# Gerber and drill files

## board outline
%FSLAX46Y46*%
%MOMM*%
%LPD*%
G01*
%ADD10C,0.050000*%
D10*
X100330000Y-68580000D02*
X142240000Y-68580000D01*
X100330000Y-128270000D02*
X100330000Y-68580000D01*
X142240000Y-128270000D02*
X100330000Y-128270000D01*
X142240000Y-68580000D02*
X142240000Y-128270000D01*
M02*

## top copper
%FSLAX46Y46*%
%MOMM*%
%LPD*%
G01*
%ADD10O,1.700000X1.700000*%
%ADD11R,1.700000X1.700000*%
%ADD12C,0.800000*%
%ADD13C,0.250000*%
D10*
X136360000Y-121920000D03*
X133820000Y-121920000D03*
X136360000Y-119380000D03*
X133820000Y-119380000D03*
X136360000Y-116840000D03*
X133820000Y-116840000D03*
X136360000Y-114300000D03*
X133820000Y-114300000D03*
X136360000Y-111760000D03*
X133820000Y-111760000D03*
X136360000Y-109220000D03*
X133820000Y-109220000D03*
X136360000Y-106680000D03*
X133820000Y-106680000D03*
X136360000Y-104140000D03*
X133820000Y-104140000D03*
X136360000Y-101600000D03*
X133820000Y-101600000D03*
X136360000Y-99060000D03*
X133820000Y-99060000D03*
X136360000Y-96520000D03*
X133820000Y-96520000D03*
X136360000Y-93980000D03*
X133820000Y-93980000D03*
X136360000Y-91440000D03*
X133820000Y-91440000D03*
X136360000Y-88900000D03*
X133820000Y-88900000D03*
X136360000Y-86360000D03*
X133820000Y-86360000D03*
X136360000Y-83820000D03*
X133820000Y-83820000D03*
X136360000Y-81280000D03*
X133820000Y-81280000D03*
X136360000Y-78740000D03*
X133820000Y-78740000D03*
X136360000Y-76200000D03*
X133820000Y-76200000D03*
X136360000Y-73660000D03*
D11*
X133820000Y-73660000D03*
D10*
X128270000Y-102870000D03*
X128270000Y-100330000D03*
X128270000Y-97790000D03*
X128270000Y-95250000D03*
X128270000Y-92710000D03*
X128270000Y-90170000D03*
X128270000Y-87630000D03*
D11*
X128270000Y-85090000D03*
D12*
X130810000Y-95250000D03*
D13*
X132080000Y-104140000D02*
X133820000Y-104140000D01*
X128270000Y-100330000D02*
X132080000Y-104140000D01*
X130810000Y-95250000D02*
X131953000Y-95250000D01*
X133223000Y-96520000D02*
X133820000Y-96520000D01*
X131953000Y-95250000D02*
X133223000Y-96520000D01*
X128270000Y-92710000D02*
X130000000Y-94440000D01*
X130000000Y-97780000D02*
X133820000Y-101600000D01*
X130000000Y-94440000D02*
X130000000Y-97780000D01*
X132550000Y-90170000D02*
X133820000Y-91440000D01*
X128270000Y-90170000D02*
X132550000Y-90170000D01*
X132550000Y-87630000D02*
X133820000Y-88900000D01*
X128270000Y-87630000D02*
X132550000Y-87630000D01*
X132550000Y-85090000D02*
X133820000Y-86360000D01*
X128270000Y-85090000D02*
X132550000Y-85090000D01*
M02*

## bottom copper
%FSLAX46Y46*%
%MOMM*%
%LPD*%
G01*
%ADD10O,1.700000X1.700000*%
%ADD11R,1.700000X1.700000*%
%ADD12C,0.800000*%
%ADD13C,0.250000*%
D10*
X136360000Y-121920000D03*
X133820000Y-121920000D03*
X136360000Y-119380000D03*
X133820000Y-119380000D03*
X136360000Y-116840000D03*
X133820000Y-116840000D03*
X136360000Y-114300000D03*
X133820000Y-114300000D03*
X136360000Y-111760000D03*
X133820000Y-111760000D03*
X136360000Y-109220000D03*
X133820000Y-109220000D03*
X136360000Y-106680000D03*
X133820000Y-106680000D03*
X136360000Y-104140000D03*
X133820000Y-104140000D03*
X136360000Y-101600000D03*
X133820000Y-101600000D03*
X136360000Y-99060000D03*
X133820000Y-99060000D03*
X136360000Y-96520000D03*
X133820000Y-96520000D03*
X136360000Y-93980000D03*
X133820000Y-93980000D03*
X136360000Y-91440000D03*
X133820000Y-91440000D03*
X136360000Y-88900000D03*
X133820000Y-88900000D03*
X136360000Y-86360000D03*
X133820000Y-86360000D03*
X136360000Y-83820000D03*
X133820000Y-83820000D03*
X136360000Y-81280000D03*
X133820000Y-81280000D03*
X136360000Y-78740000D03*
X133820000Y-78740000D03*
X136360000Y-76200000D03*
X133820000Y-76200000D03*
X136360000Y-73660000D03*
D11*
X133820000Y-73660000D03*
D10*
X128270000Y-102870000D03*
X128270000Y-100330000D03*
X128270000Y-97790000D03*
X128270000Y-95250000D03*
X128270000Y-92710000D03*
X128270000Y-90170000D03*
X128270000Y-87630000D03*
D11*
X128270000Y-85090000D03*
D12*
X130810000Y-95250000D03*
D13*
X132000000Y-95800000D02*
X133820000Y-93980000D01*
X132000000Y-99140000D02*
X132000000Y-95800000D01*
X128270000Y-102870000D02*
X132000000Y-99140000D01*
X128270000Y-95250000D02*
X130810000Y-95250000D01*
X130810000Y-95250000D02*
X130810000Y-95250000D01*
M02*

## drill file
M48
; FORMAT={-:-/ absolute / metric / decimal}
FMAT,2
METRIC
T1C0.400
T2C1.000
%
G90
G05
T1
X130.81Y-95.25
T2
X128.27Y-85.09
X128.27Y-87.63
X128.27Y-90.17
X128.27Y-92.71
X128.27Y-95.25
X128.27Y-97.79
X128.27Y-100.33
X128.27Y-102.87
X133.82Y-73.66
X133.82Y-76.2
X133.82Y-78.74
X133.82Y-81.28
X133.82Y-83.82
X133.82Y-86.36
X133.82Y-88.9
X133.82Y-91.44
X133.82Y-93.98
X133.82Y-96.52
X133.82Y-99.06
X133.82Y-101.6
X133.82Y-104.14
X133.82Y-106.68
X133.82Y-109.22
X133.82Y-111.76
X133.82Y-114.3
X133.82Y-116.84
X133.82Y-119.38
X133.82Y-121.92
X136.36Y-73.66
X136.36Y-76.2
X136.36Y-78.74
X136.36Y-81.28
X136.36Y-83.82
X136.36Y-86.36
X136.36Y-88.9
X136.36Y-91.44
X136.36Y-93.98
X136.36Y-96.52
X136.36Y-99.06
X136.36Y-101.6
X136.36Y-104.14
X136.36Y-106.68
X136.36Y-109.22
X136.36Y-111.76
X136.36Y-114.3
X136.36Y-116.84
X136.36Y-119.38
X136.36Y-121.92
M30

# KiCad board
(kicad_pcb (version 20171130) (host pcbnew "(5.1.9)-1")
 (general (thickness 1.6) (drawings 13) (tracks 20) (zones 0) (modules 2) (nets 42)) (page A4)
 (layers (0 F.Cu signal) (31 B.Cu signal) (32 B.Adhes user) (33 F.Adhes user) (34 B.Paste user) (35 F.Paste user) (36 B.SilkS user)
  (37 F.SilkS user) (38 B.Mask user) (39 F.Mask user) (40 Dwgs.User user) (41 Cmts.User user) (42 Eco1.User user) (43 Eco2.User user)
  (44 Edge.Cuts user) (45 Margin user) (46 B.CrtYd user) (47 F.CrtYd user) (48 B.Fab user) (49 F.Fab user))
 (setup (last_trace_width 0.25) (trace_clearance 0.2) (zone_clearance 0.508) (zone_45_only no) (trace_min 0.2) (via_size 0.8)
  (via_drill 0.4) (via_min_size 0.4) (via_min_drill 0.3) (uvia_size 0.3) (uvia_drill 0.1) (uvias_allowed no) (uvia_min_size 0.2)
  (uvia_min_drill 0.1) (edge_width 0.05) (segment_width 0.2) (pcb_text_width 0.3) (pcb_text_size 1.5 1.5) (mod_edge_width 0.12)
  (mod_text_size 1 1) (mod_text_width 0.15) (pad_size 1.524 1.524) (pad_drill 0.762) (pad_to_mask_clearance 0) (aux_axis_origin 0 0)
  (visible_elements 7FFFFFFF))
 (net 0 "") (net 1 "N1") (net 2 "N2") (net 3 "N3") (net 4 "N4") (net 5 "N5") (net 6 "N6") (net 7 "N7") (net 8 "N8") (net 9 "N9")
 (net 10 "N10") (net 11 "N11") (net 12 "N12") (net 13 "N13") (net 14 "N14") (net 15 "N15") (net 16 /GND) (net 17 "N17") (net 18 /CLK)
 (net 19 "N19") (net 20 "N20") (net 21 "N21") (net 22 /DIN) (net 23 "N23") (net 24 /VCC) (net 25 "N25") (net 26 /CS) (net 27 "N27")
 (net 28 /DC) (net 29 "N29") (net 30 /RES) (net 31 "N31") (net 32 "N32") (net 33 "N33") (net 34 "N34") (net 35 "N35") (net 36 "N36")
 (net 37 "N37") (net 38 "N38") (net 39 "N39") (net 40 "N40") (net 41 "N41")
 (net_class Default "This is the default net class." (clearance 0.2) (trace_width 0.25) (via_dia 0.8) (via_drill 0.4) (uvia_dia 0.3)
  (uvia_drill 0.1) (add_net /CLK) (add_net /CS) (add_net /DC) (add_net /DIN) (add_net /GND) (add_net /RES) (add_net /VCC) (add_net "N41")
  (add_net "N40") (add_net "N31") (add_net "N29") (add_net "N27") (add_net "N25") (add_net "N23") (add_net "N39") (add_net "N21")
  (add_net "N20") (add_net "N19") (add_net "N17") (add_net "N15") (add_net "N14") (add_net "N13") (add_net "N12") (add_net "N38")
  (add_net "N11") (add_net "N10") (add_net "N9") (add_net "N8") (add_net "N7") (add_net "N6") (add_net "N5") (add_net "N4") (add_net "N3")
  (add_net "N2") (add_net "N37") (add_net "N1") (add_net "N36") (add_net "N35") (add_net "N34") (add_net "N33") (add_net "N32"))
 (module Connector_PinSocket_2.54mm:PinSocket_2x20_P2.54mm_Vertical (layer B.Cu) (at 133.82 73.66 180)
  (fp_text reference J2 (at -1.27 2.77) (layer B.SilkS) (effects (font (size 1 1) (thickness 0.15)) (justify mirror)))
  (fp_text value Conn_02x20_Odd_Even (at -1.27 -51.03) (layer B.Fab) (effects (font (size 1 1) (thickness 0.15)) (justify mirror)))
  (pad 40 thru_hole oval (at -2.54 -48.26 180) (size 1.7 1.7) (drill 1) (layers *.Cu *.Mask) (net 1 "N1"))
  (pad 39 thru_hole oval (at 0 -48.26 180) (size 1.7 1.7) (drill 1) (layers *.Cu *.Mask) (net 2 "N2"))
  (pad 38 thru_hole oval (at -2.54 -45.72 180) (size 1.7 1.7) (drill 1) (layers *.Cu *.Mask) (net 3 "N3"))
  (pad 37 thru_hole oval (at 0 -45.72 180) (size 1.7 1.7) (drill 1) (layers *.Cu *.Mask) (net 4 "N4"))
  (pad 36 thru_hole oval (at -2.54 -43.18 180) (size 1.7 1.7) (drill 1) (layers *.Cu *.Mask) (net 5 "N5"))
  (pad 35 thru_hole oval (at 0 -43.18 180) (size 1.7 1.7) (drill 1) (layers *.Cu *.Mask) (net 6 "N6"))
  (pad 34 thru_hole oval (at -2.54 -40.64 180) (size 1.7 1.7) (drill 1) (layers *.Cu *.Mask) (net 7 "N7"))
  (pad 33 thru_hole oval (at 0 -40.64 180) (size 1.7 1.7) (drill 1) (layers *.Cu *.Mask) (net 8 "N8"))
  (pad 32 thru_hole oval (at -2.54 -38.1 180) (size 1.7 1.7) (drill 1) (layers *.Cu *.Mask) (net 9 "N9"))
  (pad 31 thru_hole oval (at 0 -38.1 180) (size 1.7 1.7) (drill 1) (layers *.Cu *.Mask) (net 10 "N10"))
  (pad 30 thru_hole oval (at -2.54 -35.56 180) (size 1.7 1.7) (drill 1) (layers *.Cu *.Mask) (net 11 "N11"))
  (pad 29 thru_hole oval (at 0 -35.56 180) (size 1.7 1.7) (drill 1) (layers *.Cu *.Mask) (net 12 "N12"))
  (pad 28 thru_hole oval (at -2.54 -33.02 180) (size 1.7 1.7) (drill 1) (layers *.Cu *.Mask) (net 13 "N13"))
  (pad 27 thru_hole oval (at 0 -33.02 180) (size 1.7 1.7) (drill 1) (layers *.Cu *.Mask) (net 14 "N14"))
  (pad 26 thru_hole oval (at -2.54 -30.48 180) (size 1.7 1.7) (drill 1) (layers *.Cu *.Mask) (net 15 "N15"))
  (pad 25 thru_hole oval (at 0 -30.48 180) (size 1.7 1.7) (drill 1) (layers *.Cu *.Mask) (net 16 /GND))
  (pad 24 thru_hole oval (at -2.54 -27.94 180) (size 1.7 1.7) (drill 1) (layers *.Cu *.Mask) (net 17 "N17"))
  (pad 23 thru_hole oval (at 0 -27.94 180) (size 1.7 1.7) (drill 1) (layers *.Cu *.Mask) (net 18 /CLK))
  (pad 22 thru_hole oval (at -2.54 -25.4 180) (size 1.7 1.7) (drill 1) (layers *.Cu *.Mask) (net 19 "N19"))
  (pad 21 thru_hole oval (at 0 -25.4 180) (size 1.7 1.7) (drill 1) (layers *.Cu *.Mask) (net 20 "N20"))
  (pad 20 thru_hole oval (at -2.54 -22.86 180) (size 1.7 1.7) (drill 1) (layers *.Cu *.Mask) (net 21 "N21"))
  (pad 19 thru_hole oval (at 0 -22.86 180) (size 1.7 1.7) (drill 1) (layers *.Cu *.Mask) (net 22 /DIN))
  (pad 18 thru_hole oval (at -2.54 -20.32 180) (size 1.7 1.7) (drill 1) (layers *.Cu *.Mask) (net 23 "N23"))
  (pad 17 thru_hole oval (at 0 -20.32 180) (size 1.7 1.7) (drill 1) (layers *.Cu *.Mask) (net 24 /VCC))
  (pad 16 thru_hole oval (at -2.54 -17.78 180) (size 1.7 1.7) (drill 1) (layers *.Cu *.Mask) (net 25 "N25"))
  (pad 15 thru_hole oval (at 0 -17.78 180) (size 1.7 1.7) (drill 1) (layers *.Cu *.Mask) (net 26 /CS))
  (pad 14 thru_hole oval (at -2.54 -15.24 180) (size 1.7 1.7) (drill 1) (layers *.Cu *.Mask) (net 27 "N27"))
  (pad 13 thru_hole oval (at 0 -15.24 180) (size 1.7 1.7) (drill 1) (layers *.Cu *.Mask) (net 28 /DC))
  (pad 12 thru_hole oval (at -2.54 -12.7 180) (size 1.7 1.7) (drill 1) (layers *.Cu *.Mask) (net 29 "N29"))
  (pad 11 thru_hole oval (at 0 -12.7 180) (size 1.7 1.7) (drill 1) (layers *.Cu *.Mask) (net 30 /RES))
  (pad 10 thru_hole oval (at -2.54 -10.16 180) (size 1.7 1.7) (drill 1) (layers *.Cu *.Mask) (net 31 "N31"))
  (pad 9 thru_hole oval (at 0 -10.16 180) (size 1.7 1.7) (drill 1) (layers *.Cu *.Mask) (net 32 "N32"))
  (pad 8 thru_hole oval (at -2.54 -7.62 180) (size 1.7 1.7) (drill 1) (layers *.Cu *.Mask) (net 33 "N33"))
  (pad 7 thru_hole oval (at 0 -7.62 180) (size 1.7 1.7) (drill 1) (layers *.Cu *.Mask) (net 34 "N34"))
  (pad 6 thru_hole oval (at -2.54 -5.08 180) (size 1.7 1.7) (drill 1) (layers *.Cu *.Mask) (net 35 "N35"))
  (pad 5 thru_hole oval (at 0 -5.08 180) (size 1.7 1.7) (drill 1) (layers *.Cu *.Mask) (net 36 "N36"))
  (pad 4 thru_hole oval (at -2.54 -2.54 180) (size 1.7 1.7) (drill 1) (layers *.Cu *.Mask) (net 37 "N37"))
  (pad 3 thru_hole oval (at 0 -2.54 180) (size 1.7 1.7) (drill 1) (layers *.Cu *.Mask) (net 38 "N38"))
  (pad 2 thru_hole oval (at -2.54 0 180) (size 1.7 1.7) (drill 1) (layers *.Cu *.Mask) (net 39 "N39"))
  (pad 1 thru_hole rect (at 0 0 180) (size 1.7 1.7) (drill 1) (layers *.Cu *.Mask) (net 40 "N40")))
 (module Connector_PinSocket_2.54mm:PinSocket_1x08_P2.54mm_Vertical (layer F.Cu) (at 128.27 85.09)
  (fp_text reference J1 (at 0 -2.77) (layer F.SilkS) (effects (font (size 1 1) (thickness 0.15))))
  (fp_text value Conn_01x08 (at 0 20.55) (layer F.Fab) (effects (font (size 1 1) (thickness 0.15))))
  (pad 8 thru_hole oval (at 0 17.78) (size 1.7 1.7) (drill 1) (layers *.Cu *.Mask) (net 24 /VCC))
  (pad 7 thru_hole oval (at 0 15.24) (size 1.7 1.7) (drill 1) (layers *.Cu *.Mask) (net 16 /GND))
  (pad 6 thru_hole oval (at 0 12.7) (size 1.7 1.7) (drill 1) (layers *.Cu *.Mask) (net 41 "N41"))
  (pad 5 thru_hole oval (at 0 10.16) (size 1.7 1.7) (drill 1) (layers *.Cu *.Mask) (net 22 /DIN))
  (pad 4 thru_hole oval (at 0 7.62) (size 1.7 1.7) (drill 1) (layers *.Cu *.Mask) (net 18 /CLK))
  (pad 3 thru_hole oval (at 0 5.08) (size 1.7 1.7) (drill 1) (layers *.Cu *.Mask) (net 26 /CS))
  (pad 2 thru_hole oval (at 0 2.54) (size 1.7 1.7) (drill 1) (layers *.Cu *.Mask) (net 28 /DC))
  (pad 1 thru_hole rect (at 0 0) (size 1.7 1.7) (drill 1) (layers *.Cu *.Mask) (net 30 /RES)))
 (gr_line (start 100.33 68.58) (end 142.24 68.58) (layer Edge.Cuts) (width 0.05))
 (gr_line (start 100.33 128.27) (end 100.33 68.58) (layer Edge.Cuts) (width 0.05))
 (gr_line (start 142.24 128.27) (end 100.33 128.27) (layer Edge.Cuts) (width 0.05))
 (gr_line (start 142.24 68.58) (end 142.24 128.27) (layer Edge.Cuts) (width 0.05))
 (segment (start 132 95.8) (end 133.82 93.98) (width 0.25) (layer B.Cu) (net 24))
 (segment (start 132 99.14) (end 132 95.8) (width 0.25) (layer B.Cu) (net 24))
 (segment (start 128.27 102.87) (end 132 99.14) (width 0.25) (layer B.Cu) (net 24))
 (segment (start 132.08 104.14) (end 133.82 104.14) (width 0.25) (layer F.Cu) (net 16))
 (segment (start 128.27 100.33) (end 132.08 104.14) (width 0.25) (layer F.Cu) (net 16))
 (segment (start 128.27 95.25) (end 130.81 95.25) (width 0.25) (layer B.Cu) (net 22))
 (segment (start 130.81 95.25) (end 130.81 95.25) (width 0.25) (layer B.Cu) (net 22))
 (via (at 130.81 95.25) (size 0.8) (drill 0.4) (layers F.Cu B.Cu) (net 22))
 (segment (start 130.81 95.25) (end 131.953 95.25) (width 0.25) (layer F.Cu) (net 22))
 (segment (start 133.223 96.52) (end 133.82 96.52) (width 0.25) (layer F.Cu) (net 22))
 (segment (start 131.953 95.25) (end 133.223 96.52) (width 0.25) (layer F.Cu) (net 22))
 (segment (start 128.27 92.71) (end 130 94.44) (width 0.25) (layer F.Cu) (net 18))
 (segment (start 130 97.78) (end 133.82 101.6) (width 0.25) (layer F.Cu) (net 18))
 (segment (start 130 94.44) (end 130 97.78) (width 0.25) (layer F.Cu) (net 18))
 (segment (start 132.55 90.17) (end 133.82 91.44) (width 0.25) (layer F.Cu) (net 26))
 (segment (start 128.27 90.17) (end 132.55 90.17) (width 0.25) (layer F.Cu) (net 26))
 (segment (start 132.55 87.63) (end 133.82 88.9) (width 0.25) (layer F.Cu) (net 28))
 (segment (start 128.27 87.63) (end 132.55 87.63) (width 0.25) (layer F.Cu) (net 28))
 (segment (start 132.55 85.09) (end 133.82 86.36) (width 0.25) (layer F.Cu) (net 30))
 (segment (start 128.27 85.09) (end 132.55 85.09) (width 0.25) (layer F.Cu) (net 30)))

